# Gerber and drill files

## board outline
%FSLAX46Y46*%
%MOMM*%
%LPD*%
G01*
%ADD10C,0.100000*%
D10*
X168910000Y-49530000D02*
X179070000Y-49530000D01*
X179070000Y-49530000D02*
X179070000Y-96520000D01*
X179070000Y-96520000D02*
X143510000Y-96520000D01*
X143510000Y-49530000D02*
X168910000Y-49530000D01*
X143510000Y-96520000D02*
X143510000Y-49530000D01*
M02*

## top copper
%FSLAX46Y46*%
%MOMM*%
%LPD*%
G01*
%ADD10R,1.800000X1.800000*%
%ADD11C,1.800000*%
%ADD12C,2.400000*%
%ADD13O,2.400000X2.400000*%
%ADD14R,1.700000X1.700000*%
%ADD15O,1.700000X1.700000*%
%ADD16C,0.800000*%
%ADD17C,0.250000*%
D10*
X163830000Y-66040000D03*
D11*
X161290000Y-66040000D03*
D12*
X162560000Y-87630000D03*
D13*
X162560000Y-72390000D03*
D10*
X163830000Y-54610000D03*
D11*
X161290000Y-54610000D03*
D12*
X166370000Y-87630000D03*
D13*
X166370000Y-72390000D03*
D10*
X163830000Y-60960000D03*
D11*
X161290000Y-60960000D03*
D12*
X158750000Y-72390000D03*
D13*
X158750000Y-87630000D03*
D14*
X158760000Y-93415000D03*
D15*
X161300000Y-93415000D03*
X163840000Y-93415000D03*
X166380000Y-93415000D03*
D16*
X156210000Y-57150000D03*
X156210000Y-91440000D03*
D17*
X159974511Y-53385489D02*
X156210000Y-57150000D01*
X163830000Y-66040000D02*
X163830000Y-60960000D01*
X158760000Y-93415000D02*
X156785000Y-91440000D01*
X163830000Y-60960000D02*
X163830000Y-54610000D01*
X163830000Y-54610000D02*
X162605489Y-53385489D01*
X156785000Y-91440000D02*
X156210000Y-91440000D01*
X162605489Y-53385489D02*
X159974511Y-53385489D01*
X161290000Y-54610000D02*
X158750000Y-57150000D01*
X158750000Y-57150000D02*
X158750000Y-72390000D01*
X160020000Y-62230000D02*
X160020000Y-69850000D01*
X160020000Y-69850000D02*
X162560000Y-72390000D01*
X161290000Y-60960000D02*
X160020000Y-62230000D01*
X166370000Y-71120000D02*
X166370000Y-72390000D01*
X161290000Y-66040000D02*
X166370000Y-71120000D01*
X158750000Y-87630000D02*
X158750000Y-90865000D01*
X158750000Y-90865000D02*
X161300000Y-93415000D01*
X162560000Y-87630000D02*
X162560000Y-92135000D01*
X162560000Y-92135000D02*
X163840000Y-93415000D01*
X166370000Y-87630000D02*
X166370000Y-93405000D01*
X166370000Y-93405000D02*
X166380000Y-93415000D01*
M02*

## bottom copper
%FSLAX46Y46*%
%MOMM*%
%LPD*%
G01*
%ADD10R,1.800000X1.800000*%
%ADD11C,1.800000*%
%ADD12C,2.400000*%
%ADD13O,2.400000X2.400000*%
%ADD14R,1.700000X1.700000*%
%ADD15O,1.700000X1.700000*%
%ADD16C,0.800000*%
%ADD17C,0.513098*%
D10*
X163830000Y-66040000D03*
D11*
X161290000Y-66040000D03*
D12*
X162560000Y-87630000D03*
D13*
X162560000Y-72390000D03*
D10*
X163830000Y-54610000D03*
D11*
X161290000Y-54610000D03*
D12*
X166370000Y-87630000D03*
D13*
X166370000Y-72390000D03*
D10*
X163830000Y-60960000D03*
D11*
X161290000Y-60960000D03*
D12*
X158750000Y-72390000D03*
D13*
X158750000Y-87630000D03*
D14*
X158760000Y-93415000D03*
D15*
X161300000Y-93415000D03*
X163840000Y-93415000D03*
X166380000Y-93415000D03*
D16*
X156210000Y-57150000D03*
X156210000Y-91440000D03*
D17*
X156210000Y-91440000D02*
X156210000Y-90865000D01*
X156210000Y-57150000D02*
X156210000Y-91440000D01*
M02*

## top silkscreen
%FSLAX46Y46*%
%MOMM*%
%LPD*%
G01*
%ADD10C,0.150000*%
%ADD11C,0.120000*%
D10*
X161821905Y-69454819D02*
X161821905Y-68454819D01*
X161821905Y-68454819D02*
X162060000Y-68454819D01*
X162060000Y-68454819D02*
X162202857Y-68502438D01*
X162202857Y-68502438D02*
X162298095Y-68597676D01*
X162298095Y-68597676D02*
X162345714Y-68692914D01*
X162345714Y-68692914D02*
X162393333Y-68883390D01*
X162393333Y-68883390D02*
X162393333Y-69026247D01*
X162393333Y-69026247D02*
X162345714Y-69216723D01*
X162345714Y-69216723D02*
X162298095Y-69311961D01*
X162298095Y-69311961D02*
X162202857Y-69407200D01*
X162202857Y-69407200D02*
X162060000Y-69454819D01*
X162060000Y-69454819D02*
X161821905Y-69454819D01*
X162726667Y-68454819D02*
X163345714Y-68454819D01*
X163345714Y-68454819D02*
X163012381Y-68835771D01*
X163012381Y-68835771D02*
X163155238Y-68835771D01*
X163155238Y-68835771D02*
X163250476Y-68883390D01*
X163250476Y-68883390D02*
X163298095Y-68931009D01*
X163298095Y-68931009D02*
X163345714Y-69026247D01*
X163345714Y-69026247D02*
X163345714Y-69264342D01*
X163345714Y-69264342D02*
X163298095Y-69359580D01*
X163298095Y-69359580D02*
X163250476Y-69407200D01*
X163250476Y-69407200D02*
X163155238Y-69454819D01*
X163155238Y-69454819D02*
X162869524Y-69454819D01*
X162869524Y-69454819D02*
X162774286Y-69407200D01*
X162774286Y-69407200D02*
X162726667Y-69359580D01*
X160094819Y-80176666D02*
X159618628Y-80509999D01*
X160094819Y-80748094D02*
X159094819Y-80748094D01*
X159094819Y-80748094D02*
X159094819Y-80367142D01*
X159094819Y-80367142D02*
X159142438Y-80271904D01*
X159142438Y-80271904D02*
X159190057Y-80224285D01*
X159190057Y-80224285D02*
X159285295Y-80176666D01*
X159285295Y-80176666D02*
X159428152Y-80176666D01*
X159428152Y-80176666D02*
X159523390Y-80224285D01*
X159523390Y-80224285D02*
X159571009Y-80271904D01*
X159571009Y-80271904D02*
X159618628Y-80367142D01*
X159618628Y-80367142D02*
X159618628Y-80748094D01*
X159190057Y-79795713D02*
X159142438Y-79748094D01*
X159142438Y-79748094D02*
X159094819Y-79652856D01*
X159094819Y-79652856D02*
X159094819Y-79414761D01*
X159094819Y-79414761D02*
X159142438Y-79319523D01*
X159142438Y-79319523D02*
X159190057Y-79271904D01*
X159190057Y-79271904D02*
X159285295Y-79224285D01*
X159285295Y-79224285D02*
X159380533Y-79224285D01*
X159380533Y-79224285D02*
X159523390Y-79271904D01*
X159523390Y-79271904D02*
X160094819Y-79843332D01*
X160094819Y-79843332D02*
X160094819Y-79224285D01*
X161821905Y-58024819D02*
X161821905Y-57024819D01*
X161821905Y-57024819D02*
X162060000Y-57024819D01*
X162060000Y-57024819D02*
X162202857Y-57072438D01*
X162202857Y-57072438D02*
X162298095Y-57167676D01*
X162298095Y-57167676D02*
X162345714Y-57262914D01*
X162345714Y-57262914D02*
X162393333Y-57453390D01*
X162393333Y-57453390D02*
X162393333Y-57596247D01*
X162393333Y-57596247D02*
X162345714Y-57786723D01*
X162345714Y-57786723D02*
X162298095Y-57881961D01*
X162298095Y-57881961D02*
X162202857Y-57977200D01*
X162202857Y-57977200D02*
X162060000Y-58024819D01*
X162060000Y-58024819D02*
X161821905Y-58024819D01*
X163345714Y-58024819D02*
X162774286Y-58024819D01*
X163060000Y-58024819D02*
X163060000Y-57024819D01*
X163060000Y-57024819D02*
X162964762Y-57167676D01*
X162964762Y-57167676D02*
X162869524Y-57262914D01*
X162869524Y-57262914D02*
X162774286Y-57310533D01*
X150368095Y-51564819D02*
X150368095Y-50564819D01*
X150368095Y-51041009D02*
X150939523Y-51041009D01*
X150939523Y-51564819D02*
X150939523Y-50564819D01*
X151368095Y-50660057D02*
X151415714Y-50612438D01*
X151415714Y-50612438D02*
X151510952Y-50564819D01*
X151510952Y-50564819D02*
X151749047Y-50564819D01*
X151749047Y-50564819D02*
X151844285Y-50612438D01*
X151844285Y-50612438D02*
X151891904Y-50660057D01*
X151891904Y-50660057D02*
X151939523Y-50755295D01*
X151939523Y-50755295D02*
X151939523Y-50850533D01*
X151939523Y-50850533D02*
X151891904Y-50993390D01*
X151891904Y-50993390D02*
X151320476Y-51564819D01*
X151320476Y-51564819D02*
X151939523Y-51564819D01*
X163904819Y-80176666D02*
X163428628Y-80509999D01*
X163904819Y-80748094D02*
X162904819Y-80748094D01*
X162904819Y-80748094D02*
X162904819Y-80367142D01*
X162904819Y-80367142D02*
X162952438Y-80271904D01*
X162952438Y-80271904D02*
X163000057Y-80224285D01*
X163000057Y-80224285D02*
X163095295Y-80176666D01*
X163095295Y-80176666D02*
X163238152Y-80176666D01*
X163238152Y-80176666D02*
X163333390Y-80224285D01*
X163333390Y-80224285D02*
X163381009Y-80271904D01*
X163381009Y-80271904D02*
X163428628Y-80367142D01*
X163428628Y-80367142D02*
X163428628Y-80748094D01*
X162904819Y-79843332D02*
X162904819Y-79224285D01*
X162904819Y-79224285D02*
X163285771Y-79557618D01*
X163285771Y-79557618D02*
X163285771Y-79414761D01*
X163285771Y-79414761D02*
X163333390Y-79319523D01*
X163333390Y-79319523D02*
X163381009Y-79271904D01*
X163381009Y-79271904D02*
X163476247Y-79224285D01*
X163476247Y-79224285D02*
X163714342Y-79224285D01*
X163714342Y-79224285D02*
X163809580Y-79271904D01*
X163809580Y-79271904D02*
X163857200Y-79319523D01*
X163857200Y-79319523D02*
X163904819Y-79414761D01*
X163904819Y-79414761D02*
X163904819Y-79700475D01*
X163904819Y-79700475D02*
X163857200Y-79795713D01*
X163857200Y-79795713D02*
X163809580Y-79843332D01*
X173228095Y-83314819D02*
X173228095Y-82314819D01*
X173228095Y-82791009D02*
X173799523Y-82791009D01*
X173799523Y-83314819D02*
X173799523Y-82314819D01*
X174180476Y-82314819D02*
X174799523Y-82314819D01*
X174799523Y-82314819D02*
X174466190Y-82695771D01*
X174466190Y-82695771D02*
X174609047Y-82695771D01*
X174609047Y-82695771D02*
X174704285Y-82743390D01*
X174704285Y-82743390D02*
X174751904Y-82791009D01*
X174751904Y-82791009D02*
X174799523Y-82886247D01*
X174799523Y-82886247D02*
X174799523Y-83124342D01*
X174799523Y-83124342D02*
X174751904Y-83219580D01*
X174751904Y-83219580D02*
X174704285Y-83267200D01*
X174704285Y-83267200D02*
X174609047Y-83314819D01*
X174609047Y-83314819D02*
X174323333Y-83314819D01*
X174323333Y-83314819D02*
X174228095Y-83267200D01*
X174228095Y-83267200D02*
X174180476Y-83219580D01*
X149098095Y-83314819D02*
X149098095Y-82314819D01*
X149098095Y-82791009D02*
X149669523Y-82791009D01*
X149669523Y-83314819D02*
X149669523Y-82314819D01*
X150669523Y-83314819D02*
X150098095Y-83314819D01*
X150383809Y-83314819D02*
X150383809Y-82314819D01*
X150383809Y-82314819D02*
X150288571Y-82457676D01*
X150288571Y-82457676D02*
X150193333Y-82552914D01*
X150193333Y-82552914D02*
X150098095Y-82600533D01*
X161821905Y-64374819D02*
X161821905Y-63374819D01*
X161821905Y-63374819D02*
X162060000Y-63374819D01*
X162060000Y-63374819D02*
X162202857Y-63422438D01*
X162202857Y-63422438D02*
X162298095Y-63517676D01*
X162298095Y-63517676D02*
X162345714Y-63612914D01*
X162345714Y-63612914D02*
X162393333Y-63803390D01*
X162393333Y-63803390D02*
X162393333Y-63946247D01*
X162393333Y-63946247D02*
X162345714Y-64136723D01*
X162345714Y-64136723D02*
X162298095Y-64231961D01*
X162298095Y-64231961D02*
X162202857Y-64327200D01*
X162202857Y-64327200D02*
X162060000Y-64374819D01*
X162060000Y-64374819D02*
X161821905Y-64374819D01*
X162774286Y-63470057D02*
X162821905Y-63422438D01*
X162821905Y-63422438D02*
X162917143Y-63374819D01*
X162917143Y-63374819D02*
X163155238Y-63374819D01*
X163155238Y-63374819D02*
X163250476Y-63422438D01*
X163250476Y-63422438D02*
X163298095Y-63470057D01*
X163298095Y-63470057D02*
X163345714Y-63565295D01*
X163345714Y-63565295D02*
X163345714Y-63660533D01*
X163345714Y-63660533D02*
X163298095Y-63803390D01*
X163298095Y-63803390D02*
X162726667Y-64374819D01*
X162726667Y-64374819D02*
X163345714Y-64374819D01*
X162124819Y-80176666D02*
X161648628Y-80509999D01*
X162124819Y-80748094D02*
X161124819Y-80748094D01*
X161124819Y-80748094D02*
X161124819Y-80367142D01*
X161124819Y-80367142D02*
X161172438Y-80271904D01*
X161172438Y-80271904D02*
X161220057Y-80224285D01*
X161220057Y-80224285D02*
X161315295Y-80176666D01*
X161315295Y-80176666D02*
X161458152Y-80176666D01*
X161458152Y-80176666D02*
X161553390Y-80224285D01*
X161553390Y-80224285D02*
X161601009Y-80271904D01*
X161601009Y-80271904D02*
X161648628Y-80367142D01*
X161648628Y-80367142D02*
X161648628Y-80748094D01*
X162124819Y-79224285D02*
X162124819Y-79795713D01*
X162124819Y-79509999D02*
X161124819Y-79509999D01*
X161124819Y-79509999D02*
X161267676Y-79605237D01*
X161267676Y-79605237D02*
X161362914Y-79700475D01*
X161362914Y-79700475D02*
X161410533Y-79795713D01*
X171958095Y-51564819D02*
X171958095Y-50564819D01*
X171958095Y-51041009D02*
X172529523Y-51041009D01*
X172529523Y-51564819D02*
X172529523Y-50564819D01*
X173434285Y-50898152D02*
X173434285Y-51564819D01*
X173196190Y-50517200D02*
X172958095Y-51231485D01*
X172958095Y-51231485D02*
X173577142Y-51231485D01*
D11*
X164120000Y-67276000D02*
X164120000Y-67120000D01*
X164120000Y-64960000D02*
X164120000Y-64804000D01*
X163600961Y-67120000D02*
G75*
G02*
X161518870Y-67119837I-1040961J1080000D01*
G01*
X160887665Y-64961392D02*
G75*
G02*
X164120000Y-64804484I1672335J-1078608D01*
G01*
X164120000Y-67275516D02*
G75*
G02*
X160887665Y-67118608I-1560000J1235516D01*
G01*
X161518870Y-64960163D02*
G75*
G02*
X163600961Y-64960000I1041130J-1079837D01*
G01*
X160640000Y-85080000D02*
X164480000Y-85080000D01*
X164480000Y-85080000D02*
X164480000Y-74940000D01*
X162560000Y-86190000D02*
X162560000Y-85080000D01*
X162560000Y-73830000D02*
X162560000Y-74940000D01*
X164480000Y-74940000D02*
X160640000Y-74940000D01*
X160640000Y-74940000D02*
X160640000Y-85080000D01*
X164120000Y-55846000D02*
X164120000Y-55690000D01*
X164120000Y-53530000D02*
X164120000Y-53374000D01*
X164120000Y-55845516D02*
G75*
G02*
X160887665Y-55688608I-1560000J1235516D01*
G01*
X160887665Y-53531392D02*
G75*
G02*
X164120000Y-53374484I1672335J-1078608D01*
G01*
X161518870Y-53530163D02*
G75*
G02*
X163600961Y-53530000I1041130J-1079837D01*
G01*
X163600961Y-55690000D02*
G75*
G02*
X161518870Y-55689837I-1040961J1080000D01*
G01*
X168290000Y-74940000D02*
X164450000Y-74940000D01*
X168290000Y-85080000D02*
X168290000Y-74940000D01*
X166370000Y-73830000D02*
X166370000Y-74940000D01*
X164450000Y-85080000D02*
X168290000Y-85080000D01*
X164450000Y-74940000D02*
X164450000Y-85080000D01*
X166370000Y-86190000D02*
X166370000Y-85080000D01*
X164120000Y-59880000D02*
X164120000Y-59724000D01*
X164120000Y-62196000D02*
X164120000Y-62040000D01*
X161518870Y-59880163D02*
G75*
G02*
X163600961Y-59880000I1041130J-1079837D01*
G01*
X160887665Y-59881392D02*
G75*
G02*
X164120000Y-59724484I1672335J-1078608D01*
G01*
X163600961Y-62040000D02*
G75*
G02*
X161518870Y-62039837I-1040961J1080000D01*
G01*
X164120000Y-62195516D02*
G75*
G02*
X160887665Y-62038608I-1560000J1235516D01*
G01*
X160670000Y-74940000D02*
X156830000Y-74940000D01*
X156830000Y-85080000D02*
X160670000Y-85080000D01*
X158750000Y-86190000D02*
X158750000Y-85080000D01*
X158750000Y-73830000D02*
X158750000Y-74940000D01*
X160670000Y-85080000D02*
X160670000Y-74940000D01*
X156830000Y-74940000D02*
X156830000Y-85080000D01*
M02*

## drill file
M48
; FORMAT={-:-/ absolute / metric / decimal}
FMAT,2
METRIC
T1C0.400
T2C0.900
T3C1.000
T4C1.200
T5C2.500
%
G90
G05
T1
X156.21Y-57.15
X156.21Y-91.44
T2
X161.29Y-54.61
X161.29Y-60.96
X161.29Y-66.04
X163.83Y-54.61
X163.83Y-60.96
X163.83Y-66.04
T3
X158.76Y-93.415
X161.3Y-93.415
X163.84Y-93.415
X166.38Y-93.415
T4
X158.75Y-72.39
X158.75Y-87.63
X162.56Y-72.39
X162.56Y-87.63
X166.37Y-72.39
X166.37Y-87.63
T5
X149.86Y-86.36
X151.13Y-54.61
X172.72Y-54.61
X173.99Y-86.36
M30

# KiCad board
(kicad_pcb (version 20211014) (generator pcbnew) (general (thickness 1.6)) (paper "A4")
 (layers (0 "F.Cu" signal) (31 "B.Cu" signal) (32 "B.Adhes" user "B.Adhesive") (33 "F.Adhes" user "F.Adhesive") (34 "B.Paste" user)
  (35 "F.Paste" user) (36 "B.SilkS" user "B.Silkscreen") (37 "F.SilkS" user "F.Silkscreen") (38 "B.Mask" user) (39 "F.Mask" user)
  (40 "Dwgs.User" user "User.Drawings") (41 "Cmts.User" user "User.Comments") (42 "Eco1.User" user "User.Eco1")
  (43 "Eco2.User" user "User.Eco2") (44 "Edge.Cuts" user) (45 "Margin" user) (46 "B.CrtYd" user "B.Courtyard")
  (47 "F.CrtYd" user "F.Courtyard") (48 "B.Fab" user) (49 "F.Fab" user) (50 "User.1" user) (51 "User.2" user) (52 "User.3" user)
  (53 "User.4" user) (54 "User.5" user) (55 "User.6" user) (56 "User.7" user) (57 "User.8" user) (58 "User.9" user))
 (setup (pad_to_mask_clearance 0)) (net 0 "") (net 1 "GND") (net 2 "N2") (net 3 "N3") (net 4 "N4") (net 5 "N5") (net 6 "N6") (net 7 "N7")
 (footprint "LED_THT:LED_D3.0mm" (layer "F.Cu") (at 163.83 66.04 180)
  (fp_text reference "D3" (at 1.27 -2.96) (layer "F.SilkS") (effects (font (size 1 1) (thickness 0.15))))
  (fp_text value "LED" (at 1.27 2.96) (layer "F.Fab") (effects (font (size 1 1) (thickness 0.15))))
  (fp_line (start -0.29 -1.236) (end -0.29 -1.08) (layer "F.SilkS") (width 0.12))
  (fp_line (start -0.29 1.08) (end -0.29 1.236) (layer "F.SilkS") (width 0.12))
  (fp_arc (start 0.229039 -1.08) (mid 1.270117 -1.5) (end 2.31113 -1.079837) (layer "F.SilkS") (width 0.12))
  (fp_arc (start 2.942335 1.078608) (mid 1.366487 1.987659) (end -0.29 1.235516) (layer "F.SilkS") (width 0.12))
  (fp_arc (start -0.29 -1.235516) (mid 1.366487 -1.987659) (end 2.942335 -1.078608) (layer "F.SilkS") (width 0.12))
  (fp_arc (start 2.31113 1.079837) (mid 1.270117 1.5) (end 0.229039 1.08) (layer "F.SilkS") (width 0.12))
  (pad "1" thru_hole rect (at 0 0 180) (size 1.8 1.8) (drill 0.9) (layers *.Cu *.Mask) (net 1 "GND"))
  (pad "2" thru_hole circle (at 2.54 0 180) (size 1.8 1.8) (drill 0.9) (layers *.Cu *.Mask) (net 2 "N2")))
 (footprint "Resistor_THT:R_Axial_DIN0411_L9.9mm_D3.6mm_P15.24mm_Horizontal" (layer "F.Cu") (at 162.56 87.63 90)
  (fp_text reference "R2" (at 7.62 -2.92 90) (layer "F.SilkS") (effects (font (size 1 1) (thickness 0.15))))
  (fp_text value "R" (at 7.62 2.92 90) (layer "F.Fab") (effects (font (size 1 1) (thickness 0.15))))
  (fp_line (start 2.55 -1.92) (end 2.55 1.92) (layer "F.SilkS") (width 0.12))
  (fp_line (start 2.55 1.92) (end 12.69 1.92) (layer "F.SilkS") (width 0.12))
  (fp_line (start 1.44 0) (end 2.55 0) (layer "F.SilkS") (width 0.12))
  (fp_line (start 13.8 0) (end 12.69 0) (layer "F.SilkS") (width 0.12))
  (fp_line (start 12.69 1.92) (end 12.69 -1.92) (layer "F.SilkS") (width 0.12))
  (fp_line (start 12.69 -1.92) (end 2.55 -1.92) (layer "F.SilkS") (width 0.12))
  (pad "1" thru_hole circle (at 0 0 90) (size 2.4 2.4) (drill 1.2) (layers *.Cu *.Mask) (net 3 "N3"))
  (pad "2" thru_hole oval (at 15.24 0 90) (size 2.4 2.4) (drill 1.2) (layers *.Cu *.Mask) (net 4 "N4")))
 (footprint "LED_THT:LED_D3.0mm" (layer "F.Cu") (at 163.83 54.61 180)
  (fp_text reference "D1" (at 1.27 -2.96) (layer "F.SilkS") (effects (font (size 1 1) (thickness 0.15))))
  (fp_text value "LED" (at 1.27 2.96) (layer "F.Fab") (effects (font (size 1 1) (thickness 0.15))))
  (fp_line (start -0.29 -1.236) (end -0.29 -1.08) (layer "F.SilkS") (width 0.12))
  (fp_line (start -0.29 1.08) (end -0.29 1.236) (layer "F.SilkS") (width 0.12))
  (fp_arc (start -0.29 -1.235516) (mid 1.366487 -1.987659) (end 2.942335 -1.078608) (layer "F.SilkS") (width 0.12))
  (fp_arc (start 2.942335 1.078608) (mid 1.366487 1.987659) (end -0.29 1.235516) (layer "F.SilkS") (width 0.12))
  (fp_arc (start 2.31113 1.079837) (mid 1.270117 1.5) (end 0.229039 1.08) (layer "F.SilkS") (width 0.12))
  (fp_arc (start 0.229039 -1.08) (mid 1.270117 -1.5) (end 2.31113 -1.079837) (layer "F.SilkS") (width 0.12))
  (pad "1" thru_hole rect (at 0 0 180) (size 1.8 1.8) (drill 0.9) (layers *.Cu *.Mask) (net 1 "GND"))
  (pad "2" thru_hole circle (at 2.54 0 180) (size 1.8 1.8) (drill 0.9) (layers *.Cu *.Mask) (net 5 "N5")))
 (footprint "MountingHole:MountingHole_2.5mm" (layer "F.Cu") (at 151.13 54.61)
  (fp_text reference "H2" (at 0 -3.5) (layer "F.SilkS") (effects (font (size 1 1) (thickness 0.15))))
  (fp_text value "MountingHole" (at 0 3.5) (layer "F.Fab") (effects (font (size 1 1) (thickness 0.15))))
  (pad "" np_thru_hole circle (at 0 0) (size 2.5 2.5) (drill 2.5) (layers *.Cu *.Mask)))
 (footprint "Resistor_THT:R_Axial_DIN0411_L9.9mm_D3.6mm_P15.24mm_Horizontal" (layer "F.Cu") (at 166.37 87.63 90)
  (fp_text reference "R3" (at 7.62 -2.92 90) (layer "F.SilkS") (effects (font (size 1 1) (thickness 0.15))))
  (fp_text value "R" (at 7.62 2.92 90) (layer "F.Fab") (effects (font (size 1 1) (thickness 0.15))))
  (fp_line (start 12.69 1.92) (end 12.69 -1.92) (layer "F.SilkS") (width 0.12))
  (fp_line (start 2.55 1.92) (end 12.69 1.92) (layer "F.SilkS") (width 0.12))
  (fp_line (start 13.8 0) (end 12.69 0) (layer "F.SilkS") (width 0.12))
  (fp_line (start 2.55 -1.92) (end 2.55 1.92) (layer "F.SilkS") (width 0.12))
  (fp_line (start 12.69 -1.92) (end 2.55 -1.92) (layer "F.SilkS") (width 0.12))
  (fp_line (start 1.44 0) (end 2.55 0) (layer "F.SilkS") (width 0.12))
  (pad "1" thru_hole circle (at 0 0 90) (size 2.4 2.4) (drill 1.2) (layers *.Cu *.Mask) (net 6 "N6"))
  (pad "2" thru_hole oval (at 15.24 0 90) (size 2.4 2.4) (drill 1.2) (layers *.Cu *.Mask) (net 2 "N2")))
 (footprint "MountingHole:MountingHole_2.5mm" (layer "F.Cu") (at 173.99 86.36)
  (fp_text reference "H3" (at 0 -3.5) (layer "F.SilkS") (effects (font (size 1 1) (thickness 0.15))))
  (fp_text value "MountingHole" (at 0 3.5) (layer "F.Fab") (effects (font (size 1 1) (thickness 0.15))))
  (pad "" np_thru_hole circle (at 0 0) (size 2.5 2.5) (drill 2.5) (layers *.Cu *.Mask)))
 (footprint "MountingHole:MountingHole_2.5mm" (layer "F.Cu") (at 149.86 86.36)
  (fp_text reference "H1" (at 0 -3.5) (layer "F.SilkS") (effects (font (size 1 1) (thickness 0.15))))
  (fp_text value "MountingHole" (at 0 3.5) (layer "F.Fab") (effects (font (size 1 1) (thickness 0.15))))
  (pad "" np_thru_hole circle (at 0 0) (size 2.5 2.5) (drill 2.5) (layers *.Cu *.Mask)))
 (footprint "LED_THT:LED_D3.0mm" (layer "F.Cu") (at 163.83 60.96 180)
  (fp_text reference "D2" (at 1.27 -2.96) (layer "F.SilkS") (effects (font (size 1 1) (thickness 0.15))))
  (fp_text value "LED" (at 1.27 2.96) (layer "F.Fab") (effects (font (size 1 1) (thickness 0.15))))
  (fp_line (start -0.29 1.08) (end -0.29 1.236) (layer "F.SilkS") (width 0.12))
  (fp_line (start -0.29 -1.236) (end -0.29 -1.08) (layer "F.SilkS") (width 0.12))
  (fp_arc (start 2.31113 1.079837) (mid 1.270117 1.5) (end 0.229039 1.08) (layer "F.SilkS") (width 0.12))
  (fp_arc (start 2.942335 1.078608) (mid 1.366487 1.987659) (end -0.29 1.235516) (layer "F.SilkS") (width 0.12))
  (fp_arc (start 0.229039 -1.08) (mid 1.270117 -1.5) (end 2.31113 -1.079837) (layer "F.SilkS") (width 0.12))
  (fp_arc (start -0.29 -1.235516) (mid 1.366487 -1.987659) (end 2.942335 -1.078608) (layer "F.SilkS") (width 0.12))
  (pad "1" thru_hole rect (at 0 0 180) (size 1.8 1.8) (drill 0.9) (layers *.Cu *.Mask) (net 1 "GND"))
  (pad "2" thru_hole circle (at 2.54 0 180) (size 1.8 1.8) (drill 0.9) (layers *.Cu *.Mask) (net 4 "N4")))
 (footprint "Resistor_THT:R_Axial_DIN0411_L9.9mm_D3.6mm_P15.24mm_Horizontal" (layer "F.Cu") (at 158.75 72.39 -90)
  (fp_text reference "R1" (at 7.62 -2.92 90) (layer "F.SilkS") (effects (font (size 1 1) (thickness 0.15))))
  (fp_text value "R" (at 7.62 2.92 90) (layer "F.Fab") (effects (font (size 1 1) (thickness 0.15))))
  (fp_line (start 2.55 -1.92) (end 2.55 1.92) (layer "F.SilkS") (width 0.12))
  (fp_line (start 12.69 1.92) (end 12.69 -1.92) (layer "F.SilkS") (width 0.12))
  (fp_line (start 13.8 0) (end 12.69 0) (layer "F.SilkS") (width 0.12))
  (fp_line (start 1.44 0) (end 2.55 0) (layer "F.SilkS") (width 0.12))
  (fp_line (start 12.69 -1.92) (end 2.55 -1.92) (layer "F.SilkS") (width 0.12))
  (fp_line (start 2.55 1.92) (end 12.69 1.92) (layer "F.SilkS") (width 0.12))
  (pad "1" thru_hole circle (at 0 0 270) (size 2.4 2.4) (drill 1.2) (layers *.Cu *.Mask) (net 5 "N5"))
  (pad "2" thru_hole oval (at 15.24 0 270) (size 2.4 2.4) (drill 1.2) (layers *.Cu *.Mask) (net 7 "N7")))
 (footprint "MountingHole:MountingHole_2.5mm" (layer "F.Cu") (at 172.72 54.61)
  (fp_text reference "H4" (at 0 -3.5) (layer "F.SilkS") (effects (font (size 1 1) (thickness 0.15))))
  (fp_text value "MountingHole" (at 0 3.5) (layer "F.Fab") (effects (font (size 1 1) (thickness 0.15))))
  (pad "" np_thru_hole circle (at 0 0) (size 2.5 2.5) (drill 2.5) (layers *.Cu *.Mask)))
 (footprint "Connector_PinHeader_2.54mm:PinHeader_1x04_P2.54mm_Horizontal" (layer "B.Cu") (at 158.76 93.415 -90)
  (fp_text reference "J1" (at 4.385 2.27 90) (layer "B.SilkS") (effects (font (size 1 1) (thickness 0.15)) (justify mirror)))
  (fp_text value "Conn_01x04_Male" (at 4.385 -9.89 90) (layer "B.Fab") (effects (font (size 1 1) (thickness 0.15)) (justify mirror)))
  (pad "1" thru_hole rect (at 0 0 270) (size 1.7 1.7) (drill 1) (layers *.Cu *.Mask) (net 1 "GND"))
  (pad "2" thru_hole oval (at 0 -2.54 270) (size 1.7 1.7) (drill 1) (layers *.Cu *.Mask) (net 7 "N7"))
  (pad "3" thru_hole oval (at 0 -5.08 270) (size 1.7 1.7) (drill 1) (layers *.Cu *.Mask) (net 3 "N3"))
  (pad "4" thru_hole oval (at 0 -7.62 270) (size 1.7 1.7) (drill 1) (layers *.Cu *.Mask) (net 6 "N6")))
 (gr_line (start 168.91 49.53) (end 179.07 49.53) (layer "Edge.Cuts") (width 0.1))
 (gr_line (start 179.07 49.53) (end 179.07 96.52) (layer "Edge.Cuts") (width 0.1))
 (gr_line (start 179.07 96.52) (end 143.51 96.52) (layer "Edge.Cuts") (width 0.1))
 (gr_line (start 143.51 49.53) (end 168.91 49.53) (layer "Edge.Cuts") (width 0.1))
 (gr_line (start 143.51 96.52) (end 143.51 49.53) (layer "Edge.Cuts") (width 0.1))
 (segment (start 159.974511 53.385489) (end 156.21 57.15) (width 0.25) (layer "F.Cu") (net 1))
 (segment (start 163.83 66.04) (end 163.83 60.96) (width 0.25) (layer "F.Cu") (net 1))
 (segment (start 158.76 93.415) (end 156.785 91.44) (width 0.25) (layer "F.Cu") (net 1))
 (segment (start 163.83 60.96) (end 163.83 54.61) (width 0.25) (layer "F.Cu") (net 1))
 (segment (start 163.83 54.61) (end 162.605489 53.385489) (width 0.25) (layer "F.Cu") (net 1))
 (segment (start 156.785 91.44) (end 156.21 91.44) (width 0.25) (layer "F.Cu") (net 1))
 (segment (start 162.605489 53.385489) (end 159.974511 53.385489) (width 0.25) (layer "F.Cu") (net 1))
 (via (at 156.21 57.15) (size 0.8) (drill 0.4) (layers "F.Cu" "B.Cu") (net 1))
 (via (at 156.21 91.44) (size 0.8) (drill 0.4) (layers "F.Cu" "B.Cu") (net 1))
 (segment (start 156.21 91.44) (end 156.21 90.865) (width 0.513098) (layer "B.Cu") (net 1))
 (segment (start 156.21 57.15) (end 156.21 91.44) (width 0.513098) (layer "B.Cu") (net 1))
 (segment (start 161.29 54.61) (end 158.75 57.15) (width 0.25) (layer "F.Cu") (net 5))
 (segment (start 158.75 57.15) (end 158.75 72.39) (width 0.25) (layer "F.Cu") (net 5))
 (segment (start 160.02 62.23) (end 160.02 69.85) (width 0.25) (layer "F.Cu") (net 4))
 (segment (start 160.02 69.85) (end 162.56 72.39) (width 0.25) (layer "F.Cu") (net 4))
 (segment (start 161.29 60.96) (end 160.02 62.23) (width 0.25) (layer "F.Cu") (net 4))
 (segment (start 166.37 71.12) (end 166.37 72.39) (width 0.25) (layer "F.Cu") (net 2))
 (segment (start 161.29 66.04) (end 166.37 71.12) (width 0.25) (layer "F.Cu") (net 2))
 (segment (start 158.75 87.63) (end 158.75 90.865) (width 0.25) (layer "F.Cu") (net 7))
 (segment (start 158.75 90.865) (end 161.3 93.415) (width 0.25) (layer "F.Cu") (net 7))
 (segment (start 162.56 87.63) (end 162.56 92.135) (width 0.25) (layer "F.Cu") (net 3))
 (segment (start 162.56 92.135) (end 163.84 93.415) (width 0.25) (layer "F.Cu") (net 3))
 (segment (start 166.37 87.63) (end 166.37 93.405) (width 0.25) (layer "F.Cu") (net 6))
 (segment (start 166.37 93.405) (end 166.38 93.415) (width 0.25) (layer "F.Cu") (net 6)))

